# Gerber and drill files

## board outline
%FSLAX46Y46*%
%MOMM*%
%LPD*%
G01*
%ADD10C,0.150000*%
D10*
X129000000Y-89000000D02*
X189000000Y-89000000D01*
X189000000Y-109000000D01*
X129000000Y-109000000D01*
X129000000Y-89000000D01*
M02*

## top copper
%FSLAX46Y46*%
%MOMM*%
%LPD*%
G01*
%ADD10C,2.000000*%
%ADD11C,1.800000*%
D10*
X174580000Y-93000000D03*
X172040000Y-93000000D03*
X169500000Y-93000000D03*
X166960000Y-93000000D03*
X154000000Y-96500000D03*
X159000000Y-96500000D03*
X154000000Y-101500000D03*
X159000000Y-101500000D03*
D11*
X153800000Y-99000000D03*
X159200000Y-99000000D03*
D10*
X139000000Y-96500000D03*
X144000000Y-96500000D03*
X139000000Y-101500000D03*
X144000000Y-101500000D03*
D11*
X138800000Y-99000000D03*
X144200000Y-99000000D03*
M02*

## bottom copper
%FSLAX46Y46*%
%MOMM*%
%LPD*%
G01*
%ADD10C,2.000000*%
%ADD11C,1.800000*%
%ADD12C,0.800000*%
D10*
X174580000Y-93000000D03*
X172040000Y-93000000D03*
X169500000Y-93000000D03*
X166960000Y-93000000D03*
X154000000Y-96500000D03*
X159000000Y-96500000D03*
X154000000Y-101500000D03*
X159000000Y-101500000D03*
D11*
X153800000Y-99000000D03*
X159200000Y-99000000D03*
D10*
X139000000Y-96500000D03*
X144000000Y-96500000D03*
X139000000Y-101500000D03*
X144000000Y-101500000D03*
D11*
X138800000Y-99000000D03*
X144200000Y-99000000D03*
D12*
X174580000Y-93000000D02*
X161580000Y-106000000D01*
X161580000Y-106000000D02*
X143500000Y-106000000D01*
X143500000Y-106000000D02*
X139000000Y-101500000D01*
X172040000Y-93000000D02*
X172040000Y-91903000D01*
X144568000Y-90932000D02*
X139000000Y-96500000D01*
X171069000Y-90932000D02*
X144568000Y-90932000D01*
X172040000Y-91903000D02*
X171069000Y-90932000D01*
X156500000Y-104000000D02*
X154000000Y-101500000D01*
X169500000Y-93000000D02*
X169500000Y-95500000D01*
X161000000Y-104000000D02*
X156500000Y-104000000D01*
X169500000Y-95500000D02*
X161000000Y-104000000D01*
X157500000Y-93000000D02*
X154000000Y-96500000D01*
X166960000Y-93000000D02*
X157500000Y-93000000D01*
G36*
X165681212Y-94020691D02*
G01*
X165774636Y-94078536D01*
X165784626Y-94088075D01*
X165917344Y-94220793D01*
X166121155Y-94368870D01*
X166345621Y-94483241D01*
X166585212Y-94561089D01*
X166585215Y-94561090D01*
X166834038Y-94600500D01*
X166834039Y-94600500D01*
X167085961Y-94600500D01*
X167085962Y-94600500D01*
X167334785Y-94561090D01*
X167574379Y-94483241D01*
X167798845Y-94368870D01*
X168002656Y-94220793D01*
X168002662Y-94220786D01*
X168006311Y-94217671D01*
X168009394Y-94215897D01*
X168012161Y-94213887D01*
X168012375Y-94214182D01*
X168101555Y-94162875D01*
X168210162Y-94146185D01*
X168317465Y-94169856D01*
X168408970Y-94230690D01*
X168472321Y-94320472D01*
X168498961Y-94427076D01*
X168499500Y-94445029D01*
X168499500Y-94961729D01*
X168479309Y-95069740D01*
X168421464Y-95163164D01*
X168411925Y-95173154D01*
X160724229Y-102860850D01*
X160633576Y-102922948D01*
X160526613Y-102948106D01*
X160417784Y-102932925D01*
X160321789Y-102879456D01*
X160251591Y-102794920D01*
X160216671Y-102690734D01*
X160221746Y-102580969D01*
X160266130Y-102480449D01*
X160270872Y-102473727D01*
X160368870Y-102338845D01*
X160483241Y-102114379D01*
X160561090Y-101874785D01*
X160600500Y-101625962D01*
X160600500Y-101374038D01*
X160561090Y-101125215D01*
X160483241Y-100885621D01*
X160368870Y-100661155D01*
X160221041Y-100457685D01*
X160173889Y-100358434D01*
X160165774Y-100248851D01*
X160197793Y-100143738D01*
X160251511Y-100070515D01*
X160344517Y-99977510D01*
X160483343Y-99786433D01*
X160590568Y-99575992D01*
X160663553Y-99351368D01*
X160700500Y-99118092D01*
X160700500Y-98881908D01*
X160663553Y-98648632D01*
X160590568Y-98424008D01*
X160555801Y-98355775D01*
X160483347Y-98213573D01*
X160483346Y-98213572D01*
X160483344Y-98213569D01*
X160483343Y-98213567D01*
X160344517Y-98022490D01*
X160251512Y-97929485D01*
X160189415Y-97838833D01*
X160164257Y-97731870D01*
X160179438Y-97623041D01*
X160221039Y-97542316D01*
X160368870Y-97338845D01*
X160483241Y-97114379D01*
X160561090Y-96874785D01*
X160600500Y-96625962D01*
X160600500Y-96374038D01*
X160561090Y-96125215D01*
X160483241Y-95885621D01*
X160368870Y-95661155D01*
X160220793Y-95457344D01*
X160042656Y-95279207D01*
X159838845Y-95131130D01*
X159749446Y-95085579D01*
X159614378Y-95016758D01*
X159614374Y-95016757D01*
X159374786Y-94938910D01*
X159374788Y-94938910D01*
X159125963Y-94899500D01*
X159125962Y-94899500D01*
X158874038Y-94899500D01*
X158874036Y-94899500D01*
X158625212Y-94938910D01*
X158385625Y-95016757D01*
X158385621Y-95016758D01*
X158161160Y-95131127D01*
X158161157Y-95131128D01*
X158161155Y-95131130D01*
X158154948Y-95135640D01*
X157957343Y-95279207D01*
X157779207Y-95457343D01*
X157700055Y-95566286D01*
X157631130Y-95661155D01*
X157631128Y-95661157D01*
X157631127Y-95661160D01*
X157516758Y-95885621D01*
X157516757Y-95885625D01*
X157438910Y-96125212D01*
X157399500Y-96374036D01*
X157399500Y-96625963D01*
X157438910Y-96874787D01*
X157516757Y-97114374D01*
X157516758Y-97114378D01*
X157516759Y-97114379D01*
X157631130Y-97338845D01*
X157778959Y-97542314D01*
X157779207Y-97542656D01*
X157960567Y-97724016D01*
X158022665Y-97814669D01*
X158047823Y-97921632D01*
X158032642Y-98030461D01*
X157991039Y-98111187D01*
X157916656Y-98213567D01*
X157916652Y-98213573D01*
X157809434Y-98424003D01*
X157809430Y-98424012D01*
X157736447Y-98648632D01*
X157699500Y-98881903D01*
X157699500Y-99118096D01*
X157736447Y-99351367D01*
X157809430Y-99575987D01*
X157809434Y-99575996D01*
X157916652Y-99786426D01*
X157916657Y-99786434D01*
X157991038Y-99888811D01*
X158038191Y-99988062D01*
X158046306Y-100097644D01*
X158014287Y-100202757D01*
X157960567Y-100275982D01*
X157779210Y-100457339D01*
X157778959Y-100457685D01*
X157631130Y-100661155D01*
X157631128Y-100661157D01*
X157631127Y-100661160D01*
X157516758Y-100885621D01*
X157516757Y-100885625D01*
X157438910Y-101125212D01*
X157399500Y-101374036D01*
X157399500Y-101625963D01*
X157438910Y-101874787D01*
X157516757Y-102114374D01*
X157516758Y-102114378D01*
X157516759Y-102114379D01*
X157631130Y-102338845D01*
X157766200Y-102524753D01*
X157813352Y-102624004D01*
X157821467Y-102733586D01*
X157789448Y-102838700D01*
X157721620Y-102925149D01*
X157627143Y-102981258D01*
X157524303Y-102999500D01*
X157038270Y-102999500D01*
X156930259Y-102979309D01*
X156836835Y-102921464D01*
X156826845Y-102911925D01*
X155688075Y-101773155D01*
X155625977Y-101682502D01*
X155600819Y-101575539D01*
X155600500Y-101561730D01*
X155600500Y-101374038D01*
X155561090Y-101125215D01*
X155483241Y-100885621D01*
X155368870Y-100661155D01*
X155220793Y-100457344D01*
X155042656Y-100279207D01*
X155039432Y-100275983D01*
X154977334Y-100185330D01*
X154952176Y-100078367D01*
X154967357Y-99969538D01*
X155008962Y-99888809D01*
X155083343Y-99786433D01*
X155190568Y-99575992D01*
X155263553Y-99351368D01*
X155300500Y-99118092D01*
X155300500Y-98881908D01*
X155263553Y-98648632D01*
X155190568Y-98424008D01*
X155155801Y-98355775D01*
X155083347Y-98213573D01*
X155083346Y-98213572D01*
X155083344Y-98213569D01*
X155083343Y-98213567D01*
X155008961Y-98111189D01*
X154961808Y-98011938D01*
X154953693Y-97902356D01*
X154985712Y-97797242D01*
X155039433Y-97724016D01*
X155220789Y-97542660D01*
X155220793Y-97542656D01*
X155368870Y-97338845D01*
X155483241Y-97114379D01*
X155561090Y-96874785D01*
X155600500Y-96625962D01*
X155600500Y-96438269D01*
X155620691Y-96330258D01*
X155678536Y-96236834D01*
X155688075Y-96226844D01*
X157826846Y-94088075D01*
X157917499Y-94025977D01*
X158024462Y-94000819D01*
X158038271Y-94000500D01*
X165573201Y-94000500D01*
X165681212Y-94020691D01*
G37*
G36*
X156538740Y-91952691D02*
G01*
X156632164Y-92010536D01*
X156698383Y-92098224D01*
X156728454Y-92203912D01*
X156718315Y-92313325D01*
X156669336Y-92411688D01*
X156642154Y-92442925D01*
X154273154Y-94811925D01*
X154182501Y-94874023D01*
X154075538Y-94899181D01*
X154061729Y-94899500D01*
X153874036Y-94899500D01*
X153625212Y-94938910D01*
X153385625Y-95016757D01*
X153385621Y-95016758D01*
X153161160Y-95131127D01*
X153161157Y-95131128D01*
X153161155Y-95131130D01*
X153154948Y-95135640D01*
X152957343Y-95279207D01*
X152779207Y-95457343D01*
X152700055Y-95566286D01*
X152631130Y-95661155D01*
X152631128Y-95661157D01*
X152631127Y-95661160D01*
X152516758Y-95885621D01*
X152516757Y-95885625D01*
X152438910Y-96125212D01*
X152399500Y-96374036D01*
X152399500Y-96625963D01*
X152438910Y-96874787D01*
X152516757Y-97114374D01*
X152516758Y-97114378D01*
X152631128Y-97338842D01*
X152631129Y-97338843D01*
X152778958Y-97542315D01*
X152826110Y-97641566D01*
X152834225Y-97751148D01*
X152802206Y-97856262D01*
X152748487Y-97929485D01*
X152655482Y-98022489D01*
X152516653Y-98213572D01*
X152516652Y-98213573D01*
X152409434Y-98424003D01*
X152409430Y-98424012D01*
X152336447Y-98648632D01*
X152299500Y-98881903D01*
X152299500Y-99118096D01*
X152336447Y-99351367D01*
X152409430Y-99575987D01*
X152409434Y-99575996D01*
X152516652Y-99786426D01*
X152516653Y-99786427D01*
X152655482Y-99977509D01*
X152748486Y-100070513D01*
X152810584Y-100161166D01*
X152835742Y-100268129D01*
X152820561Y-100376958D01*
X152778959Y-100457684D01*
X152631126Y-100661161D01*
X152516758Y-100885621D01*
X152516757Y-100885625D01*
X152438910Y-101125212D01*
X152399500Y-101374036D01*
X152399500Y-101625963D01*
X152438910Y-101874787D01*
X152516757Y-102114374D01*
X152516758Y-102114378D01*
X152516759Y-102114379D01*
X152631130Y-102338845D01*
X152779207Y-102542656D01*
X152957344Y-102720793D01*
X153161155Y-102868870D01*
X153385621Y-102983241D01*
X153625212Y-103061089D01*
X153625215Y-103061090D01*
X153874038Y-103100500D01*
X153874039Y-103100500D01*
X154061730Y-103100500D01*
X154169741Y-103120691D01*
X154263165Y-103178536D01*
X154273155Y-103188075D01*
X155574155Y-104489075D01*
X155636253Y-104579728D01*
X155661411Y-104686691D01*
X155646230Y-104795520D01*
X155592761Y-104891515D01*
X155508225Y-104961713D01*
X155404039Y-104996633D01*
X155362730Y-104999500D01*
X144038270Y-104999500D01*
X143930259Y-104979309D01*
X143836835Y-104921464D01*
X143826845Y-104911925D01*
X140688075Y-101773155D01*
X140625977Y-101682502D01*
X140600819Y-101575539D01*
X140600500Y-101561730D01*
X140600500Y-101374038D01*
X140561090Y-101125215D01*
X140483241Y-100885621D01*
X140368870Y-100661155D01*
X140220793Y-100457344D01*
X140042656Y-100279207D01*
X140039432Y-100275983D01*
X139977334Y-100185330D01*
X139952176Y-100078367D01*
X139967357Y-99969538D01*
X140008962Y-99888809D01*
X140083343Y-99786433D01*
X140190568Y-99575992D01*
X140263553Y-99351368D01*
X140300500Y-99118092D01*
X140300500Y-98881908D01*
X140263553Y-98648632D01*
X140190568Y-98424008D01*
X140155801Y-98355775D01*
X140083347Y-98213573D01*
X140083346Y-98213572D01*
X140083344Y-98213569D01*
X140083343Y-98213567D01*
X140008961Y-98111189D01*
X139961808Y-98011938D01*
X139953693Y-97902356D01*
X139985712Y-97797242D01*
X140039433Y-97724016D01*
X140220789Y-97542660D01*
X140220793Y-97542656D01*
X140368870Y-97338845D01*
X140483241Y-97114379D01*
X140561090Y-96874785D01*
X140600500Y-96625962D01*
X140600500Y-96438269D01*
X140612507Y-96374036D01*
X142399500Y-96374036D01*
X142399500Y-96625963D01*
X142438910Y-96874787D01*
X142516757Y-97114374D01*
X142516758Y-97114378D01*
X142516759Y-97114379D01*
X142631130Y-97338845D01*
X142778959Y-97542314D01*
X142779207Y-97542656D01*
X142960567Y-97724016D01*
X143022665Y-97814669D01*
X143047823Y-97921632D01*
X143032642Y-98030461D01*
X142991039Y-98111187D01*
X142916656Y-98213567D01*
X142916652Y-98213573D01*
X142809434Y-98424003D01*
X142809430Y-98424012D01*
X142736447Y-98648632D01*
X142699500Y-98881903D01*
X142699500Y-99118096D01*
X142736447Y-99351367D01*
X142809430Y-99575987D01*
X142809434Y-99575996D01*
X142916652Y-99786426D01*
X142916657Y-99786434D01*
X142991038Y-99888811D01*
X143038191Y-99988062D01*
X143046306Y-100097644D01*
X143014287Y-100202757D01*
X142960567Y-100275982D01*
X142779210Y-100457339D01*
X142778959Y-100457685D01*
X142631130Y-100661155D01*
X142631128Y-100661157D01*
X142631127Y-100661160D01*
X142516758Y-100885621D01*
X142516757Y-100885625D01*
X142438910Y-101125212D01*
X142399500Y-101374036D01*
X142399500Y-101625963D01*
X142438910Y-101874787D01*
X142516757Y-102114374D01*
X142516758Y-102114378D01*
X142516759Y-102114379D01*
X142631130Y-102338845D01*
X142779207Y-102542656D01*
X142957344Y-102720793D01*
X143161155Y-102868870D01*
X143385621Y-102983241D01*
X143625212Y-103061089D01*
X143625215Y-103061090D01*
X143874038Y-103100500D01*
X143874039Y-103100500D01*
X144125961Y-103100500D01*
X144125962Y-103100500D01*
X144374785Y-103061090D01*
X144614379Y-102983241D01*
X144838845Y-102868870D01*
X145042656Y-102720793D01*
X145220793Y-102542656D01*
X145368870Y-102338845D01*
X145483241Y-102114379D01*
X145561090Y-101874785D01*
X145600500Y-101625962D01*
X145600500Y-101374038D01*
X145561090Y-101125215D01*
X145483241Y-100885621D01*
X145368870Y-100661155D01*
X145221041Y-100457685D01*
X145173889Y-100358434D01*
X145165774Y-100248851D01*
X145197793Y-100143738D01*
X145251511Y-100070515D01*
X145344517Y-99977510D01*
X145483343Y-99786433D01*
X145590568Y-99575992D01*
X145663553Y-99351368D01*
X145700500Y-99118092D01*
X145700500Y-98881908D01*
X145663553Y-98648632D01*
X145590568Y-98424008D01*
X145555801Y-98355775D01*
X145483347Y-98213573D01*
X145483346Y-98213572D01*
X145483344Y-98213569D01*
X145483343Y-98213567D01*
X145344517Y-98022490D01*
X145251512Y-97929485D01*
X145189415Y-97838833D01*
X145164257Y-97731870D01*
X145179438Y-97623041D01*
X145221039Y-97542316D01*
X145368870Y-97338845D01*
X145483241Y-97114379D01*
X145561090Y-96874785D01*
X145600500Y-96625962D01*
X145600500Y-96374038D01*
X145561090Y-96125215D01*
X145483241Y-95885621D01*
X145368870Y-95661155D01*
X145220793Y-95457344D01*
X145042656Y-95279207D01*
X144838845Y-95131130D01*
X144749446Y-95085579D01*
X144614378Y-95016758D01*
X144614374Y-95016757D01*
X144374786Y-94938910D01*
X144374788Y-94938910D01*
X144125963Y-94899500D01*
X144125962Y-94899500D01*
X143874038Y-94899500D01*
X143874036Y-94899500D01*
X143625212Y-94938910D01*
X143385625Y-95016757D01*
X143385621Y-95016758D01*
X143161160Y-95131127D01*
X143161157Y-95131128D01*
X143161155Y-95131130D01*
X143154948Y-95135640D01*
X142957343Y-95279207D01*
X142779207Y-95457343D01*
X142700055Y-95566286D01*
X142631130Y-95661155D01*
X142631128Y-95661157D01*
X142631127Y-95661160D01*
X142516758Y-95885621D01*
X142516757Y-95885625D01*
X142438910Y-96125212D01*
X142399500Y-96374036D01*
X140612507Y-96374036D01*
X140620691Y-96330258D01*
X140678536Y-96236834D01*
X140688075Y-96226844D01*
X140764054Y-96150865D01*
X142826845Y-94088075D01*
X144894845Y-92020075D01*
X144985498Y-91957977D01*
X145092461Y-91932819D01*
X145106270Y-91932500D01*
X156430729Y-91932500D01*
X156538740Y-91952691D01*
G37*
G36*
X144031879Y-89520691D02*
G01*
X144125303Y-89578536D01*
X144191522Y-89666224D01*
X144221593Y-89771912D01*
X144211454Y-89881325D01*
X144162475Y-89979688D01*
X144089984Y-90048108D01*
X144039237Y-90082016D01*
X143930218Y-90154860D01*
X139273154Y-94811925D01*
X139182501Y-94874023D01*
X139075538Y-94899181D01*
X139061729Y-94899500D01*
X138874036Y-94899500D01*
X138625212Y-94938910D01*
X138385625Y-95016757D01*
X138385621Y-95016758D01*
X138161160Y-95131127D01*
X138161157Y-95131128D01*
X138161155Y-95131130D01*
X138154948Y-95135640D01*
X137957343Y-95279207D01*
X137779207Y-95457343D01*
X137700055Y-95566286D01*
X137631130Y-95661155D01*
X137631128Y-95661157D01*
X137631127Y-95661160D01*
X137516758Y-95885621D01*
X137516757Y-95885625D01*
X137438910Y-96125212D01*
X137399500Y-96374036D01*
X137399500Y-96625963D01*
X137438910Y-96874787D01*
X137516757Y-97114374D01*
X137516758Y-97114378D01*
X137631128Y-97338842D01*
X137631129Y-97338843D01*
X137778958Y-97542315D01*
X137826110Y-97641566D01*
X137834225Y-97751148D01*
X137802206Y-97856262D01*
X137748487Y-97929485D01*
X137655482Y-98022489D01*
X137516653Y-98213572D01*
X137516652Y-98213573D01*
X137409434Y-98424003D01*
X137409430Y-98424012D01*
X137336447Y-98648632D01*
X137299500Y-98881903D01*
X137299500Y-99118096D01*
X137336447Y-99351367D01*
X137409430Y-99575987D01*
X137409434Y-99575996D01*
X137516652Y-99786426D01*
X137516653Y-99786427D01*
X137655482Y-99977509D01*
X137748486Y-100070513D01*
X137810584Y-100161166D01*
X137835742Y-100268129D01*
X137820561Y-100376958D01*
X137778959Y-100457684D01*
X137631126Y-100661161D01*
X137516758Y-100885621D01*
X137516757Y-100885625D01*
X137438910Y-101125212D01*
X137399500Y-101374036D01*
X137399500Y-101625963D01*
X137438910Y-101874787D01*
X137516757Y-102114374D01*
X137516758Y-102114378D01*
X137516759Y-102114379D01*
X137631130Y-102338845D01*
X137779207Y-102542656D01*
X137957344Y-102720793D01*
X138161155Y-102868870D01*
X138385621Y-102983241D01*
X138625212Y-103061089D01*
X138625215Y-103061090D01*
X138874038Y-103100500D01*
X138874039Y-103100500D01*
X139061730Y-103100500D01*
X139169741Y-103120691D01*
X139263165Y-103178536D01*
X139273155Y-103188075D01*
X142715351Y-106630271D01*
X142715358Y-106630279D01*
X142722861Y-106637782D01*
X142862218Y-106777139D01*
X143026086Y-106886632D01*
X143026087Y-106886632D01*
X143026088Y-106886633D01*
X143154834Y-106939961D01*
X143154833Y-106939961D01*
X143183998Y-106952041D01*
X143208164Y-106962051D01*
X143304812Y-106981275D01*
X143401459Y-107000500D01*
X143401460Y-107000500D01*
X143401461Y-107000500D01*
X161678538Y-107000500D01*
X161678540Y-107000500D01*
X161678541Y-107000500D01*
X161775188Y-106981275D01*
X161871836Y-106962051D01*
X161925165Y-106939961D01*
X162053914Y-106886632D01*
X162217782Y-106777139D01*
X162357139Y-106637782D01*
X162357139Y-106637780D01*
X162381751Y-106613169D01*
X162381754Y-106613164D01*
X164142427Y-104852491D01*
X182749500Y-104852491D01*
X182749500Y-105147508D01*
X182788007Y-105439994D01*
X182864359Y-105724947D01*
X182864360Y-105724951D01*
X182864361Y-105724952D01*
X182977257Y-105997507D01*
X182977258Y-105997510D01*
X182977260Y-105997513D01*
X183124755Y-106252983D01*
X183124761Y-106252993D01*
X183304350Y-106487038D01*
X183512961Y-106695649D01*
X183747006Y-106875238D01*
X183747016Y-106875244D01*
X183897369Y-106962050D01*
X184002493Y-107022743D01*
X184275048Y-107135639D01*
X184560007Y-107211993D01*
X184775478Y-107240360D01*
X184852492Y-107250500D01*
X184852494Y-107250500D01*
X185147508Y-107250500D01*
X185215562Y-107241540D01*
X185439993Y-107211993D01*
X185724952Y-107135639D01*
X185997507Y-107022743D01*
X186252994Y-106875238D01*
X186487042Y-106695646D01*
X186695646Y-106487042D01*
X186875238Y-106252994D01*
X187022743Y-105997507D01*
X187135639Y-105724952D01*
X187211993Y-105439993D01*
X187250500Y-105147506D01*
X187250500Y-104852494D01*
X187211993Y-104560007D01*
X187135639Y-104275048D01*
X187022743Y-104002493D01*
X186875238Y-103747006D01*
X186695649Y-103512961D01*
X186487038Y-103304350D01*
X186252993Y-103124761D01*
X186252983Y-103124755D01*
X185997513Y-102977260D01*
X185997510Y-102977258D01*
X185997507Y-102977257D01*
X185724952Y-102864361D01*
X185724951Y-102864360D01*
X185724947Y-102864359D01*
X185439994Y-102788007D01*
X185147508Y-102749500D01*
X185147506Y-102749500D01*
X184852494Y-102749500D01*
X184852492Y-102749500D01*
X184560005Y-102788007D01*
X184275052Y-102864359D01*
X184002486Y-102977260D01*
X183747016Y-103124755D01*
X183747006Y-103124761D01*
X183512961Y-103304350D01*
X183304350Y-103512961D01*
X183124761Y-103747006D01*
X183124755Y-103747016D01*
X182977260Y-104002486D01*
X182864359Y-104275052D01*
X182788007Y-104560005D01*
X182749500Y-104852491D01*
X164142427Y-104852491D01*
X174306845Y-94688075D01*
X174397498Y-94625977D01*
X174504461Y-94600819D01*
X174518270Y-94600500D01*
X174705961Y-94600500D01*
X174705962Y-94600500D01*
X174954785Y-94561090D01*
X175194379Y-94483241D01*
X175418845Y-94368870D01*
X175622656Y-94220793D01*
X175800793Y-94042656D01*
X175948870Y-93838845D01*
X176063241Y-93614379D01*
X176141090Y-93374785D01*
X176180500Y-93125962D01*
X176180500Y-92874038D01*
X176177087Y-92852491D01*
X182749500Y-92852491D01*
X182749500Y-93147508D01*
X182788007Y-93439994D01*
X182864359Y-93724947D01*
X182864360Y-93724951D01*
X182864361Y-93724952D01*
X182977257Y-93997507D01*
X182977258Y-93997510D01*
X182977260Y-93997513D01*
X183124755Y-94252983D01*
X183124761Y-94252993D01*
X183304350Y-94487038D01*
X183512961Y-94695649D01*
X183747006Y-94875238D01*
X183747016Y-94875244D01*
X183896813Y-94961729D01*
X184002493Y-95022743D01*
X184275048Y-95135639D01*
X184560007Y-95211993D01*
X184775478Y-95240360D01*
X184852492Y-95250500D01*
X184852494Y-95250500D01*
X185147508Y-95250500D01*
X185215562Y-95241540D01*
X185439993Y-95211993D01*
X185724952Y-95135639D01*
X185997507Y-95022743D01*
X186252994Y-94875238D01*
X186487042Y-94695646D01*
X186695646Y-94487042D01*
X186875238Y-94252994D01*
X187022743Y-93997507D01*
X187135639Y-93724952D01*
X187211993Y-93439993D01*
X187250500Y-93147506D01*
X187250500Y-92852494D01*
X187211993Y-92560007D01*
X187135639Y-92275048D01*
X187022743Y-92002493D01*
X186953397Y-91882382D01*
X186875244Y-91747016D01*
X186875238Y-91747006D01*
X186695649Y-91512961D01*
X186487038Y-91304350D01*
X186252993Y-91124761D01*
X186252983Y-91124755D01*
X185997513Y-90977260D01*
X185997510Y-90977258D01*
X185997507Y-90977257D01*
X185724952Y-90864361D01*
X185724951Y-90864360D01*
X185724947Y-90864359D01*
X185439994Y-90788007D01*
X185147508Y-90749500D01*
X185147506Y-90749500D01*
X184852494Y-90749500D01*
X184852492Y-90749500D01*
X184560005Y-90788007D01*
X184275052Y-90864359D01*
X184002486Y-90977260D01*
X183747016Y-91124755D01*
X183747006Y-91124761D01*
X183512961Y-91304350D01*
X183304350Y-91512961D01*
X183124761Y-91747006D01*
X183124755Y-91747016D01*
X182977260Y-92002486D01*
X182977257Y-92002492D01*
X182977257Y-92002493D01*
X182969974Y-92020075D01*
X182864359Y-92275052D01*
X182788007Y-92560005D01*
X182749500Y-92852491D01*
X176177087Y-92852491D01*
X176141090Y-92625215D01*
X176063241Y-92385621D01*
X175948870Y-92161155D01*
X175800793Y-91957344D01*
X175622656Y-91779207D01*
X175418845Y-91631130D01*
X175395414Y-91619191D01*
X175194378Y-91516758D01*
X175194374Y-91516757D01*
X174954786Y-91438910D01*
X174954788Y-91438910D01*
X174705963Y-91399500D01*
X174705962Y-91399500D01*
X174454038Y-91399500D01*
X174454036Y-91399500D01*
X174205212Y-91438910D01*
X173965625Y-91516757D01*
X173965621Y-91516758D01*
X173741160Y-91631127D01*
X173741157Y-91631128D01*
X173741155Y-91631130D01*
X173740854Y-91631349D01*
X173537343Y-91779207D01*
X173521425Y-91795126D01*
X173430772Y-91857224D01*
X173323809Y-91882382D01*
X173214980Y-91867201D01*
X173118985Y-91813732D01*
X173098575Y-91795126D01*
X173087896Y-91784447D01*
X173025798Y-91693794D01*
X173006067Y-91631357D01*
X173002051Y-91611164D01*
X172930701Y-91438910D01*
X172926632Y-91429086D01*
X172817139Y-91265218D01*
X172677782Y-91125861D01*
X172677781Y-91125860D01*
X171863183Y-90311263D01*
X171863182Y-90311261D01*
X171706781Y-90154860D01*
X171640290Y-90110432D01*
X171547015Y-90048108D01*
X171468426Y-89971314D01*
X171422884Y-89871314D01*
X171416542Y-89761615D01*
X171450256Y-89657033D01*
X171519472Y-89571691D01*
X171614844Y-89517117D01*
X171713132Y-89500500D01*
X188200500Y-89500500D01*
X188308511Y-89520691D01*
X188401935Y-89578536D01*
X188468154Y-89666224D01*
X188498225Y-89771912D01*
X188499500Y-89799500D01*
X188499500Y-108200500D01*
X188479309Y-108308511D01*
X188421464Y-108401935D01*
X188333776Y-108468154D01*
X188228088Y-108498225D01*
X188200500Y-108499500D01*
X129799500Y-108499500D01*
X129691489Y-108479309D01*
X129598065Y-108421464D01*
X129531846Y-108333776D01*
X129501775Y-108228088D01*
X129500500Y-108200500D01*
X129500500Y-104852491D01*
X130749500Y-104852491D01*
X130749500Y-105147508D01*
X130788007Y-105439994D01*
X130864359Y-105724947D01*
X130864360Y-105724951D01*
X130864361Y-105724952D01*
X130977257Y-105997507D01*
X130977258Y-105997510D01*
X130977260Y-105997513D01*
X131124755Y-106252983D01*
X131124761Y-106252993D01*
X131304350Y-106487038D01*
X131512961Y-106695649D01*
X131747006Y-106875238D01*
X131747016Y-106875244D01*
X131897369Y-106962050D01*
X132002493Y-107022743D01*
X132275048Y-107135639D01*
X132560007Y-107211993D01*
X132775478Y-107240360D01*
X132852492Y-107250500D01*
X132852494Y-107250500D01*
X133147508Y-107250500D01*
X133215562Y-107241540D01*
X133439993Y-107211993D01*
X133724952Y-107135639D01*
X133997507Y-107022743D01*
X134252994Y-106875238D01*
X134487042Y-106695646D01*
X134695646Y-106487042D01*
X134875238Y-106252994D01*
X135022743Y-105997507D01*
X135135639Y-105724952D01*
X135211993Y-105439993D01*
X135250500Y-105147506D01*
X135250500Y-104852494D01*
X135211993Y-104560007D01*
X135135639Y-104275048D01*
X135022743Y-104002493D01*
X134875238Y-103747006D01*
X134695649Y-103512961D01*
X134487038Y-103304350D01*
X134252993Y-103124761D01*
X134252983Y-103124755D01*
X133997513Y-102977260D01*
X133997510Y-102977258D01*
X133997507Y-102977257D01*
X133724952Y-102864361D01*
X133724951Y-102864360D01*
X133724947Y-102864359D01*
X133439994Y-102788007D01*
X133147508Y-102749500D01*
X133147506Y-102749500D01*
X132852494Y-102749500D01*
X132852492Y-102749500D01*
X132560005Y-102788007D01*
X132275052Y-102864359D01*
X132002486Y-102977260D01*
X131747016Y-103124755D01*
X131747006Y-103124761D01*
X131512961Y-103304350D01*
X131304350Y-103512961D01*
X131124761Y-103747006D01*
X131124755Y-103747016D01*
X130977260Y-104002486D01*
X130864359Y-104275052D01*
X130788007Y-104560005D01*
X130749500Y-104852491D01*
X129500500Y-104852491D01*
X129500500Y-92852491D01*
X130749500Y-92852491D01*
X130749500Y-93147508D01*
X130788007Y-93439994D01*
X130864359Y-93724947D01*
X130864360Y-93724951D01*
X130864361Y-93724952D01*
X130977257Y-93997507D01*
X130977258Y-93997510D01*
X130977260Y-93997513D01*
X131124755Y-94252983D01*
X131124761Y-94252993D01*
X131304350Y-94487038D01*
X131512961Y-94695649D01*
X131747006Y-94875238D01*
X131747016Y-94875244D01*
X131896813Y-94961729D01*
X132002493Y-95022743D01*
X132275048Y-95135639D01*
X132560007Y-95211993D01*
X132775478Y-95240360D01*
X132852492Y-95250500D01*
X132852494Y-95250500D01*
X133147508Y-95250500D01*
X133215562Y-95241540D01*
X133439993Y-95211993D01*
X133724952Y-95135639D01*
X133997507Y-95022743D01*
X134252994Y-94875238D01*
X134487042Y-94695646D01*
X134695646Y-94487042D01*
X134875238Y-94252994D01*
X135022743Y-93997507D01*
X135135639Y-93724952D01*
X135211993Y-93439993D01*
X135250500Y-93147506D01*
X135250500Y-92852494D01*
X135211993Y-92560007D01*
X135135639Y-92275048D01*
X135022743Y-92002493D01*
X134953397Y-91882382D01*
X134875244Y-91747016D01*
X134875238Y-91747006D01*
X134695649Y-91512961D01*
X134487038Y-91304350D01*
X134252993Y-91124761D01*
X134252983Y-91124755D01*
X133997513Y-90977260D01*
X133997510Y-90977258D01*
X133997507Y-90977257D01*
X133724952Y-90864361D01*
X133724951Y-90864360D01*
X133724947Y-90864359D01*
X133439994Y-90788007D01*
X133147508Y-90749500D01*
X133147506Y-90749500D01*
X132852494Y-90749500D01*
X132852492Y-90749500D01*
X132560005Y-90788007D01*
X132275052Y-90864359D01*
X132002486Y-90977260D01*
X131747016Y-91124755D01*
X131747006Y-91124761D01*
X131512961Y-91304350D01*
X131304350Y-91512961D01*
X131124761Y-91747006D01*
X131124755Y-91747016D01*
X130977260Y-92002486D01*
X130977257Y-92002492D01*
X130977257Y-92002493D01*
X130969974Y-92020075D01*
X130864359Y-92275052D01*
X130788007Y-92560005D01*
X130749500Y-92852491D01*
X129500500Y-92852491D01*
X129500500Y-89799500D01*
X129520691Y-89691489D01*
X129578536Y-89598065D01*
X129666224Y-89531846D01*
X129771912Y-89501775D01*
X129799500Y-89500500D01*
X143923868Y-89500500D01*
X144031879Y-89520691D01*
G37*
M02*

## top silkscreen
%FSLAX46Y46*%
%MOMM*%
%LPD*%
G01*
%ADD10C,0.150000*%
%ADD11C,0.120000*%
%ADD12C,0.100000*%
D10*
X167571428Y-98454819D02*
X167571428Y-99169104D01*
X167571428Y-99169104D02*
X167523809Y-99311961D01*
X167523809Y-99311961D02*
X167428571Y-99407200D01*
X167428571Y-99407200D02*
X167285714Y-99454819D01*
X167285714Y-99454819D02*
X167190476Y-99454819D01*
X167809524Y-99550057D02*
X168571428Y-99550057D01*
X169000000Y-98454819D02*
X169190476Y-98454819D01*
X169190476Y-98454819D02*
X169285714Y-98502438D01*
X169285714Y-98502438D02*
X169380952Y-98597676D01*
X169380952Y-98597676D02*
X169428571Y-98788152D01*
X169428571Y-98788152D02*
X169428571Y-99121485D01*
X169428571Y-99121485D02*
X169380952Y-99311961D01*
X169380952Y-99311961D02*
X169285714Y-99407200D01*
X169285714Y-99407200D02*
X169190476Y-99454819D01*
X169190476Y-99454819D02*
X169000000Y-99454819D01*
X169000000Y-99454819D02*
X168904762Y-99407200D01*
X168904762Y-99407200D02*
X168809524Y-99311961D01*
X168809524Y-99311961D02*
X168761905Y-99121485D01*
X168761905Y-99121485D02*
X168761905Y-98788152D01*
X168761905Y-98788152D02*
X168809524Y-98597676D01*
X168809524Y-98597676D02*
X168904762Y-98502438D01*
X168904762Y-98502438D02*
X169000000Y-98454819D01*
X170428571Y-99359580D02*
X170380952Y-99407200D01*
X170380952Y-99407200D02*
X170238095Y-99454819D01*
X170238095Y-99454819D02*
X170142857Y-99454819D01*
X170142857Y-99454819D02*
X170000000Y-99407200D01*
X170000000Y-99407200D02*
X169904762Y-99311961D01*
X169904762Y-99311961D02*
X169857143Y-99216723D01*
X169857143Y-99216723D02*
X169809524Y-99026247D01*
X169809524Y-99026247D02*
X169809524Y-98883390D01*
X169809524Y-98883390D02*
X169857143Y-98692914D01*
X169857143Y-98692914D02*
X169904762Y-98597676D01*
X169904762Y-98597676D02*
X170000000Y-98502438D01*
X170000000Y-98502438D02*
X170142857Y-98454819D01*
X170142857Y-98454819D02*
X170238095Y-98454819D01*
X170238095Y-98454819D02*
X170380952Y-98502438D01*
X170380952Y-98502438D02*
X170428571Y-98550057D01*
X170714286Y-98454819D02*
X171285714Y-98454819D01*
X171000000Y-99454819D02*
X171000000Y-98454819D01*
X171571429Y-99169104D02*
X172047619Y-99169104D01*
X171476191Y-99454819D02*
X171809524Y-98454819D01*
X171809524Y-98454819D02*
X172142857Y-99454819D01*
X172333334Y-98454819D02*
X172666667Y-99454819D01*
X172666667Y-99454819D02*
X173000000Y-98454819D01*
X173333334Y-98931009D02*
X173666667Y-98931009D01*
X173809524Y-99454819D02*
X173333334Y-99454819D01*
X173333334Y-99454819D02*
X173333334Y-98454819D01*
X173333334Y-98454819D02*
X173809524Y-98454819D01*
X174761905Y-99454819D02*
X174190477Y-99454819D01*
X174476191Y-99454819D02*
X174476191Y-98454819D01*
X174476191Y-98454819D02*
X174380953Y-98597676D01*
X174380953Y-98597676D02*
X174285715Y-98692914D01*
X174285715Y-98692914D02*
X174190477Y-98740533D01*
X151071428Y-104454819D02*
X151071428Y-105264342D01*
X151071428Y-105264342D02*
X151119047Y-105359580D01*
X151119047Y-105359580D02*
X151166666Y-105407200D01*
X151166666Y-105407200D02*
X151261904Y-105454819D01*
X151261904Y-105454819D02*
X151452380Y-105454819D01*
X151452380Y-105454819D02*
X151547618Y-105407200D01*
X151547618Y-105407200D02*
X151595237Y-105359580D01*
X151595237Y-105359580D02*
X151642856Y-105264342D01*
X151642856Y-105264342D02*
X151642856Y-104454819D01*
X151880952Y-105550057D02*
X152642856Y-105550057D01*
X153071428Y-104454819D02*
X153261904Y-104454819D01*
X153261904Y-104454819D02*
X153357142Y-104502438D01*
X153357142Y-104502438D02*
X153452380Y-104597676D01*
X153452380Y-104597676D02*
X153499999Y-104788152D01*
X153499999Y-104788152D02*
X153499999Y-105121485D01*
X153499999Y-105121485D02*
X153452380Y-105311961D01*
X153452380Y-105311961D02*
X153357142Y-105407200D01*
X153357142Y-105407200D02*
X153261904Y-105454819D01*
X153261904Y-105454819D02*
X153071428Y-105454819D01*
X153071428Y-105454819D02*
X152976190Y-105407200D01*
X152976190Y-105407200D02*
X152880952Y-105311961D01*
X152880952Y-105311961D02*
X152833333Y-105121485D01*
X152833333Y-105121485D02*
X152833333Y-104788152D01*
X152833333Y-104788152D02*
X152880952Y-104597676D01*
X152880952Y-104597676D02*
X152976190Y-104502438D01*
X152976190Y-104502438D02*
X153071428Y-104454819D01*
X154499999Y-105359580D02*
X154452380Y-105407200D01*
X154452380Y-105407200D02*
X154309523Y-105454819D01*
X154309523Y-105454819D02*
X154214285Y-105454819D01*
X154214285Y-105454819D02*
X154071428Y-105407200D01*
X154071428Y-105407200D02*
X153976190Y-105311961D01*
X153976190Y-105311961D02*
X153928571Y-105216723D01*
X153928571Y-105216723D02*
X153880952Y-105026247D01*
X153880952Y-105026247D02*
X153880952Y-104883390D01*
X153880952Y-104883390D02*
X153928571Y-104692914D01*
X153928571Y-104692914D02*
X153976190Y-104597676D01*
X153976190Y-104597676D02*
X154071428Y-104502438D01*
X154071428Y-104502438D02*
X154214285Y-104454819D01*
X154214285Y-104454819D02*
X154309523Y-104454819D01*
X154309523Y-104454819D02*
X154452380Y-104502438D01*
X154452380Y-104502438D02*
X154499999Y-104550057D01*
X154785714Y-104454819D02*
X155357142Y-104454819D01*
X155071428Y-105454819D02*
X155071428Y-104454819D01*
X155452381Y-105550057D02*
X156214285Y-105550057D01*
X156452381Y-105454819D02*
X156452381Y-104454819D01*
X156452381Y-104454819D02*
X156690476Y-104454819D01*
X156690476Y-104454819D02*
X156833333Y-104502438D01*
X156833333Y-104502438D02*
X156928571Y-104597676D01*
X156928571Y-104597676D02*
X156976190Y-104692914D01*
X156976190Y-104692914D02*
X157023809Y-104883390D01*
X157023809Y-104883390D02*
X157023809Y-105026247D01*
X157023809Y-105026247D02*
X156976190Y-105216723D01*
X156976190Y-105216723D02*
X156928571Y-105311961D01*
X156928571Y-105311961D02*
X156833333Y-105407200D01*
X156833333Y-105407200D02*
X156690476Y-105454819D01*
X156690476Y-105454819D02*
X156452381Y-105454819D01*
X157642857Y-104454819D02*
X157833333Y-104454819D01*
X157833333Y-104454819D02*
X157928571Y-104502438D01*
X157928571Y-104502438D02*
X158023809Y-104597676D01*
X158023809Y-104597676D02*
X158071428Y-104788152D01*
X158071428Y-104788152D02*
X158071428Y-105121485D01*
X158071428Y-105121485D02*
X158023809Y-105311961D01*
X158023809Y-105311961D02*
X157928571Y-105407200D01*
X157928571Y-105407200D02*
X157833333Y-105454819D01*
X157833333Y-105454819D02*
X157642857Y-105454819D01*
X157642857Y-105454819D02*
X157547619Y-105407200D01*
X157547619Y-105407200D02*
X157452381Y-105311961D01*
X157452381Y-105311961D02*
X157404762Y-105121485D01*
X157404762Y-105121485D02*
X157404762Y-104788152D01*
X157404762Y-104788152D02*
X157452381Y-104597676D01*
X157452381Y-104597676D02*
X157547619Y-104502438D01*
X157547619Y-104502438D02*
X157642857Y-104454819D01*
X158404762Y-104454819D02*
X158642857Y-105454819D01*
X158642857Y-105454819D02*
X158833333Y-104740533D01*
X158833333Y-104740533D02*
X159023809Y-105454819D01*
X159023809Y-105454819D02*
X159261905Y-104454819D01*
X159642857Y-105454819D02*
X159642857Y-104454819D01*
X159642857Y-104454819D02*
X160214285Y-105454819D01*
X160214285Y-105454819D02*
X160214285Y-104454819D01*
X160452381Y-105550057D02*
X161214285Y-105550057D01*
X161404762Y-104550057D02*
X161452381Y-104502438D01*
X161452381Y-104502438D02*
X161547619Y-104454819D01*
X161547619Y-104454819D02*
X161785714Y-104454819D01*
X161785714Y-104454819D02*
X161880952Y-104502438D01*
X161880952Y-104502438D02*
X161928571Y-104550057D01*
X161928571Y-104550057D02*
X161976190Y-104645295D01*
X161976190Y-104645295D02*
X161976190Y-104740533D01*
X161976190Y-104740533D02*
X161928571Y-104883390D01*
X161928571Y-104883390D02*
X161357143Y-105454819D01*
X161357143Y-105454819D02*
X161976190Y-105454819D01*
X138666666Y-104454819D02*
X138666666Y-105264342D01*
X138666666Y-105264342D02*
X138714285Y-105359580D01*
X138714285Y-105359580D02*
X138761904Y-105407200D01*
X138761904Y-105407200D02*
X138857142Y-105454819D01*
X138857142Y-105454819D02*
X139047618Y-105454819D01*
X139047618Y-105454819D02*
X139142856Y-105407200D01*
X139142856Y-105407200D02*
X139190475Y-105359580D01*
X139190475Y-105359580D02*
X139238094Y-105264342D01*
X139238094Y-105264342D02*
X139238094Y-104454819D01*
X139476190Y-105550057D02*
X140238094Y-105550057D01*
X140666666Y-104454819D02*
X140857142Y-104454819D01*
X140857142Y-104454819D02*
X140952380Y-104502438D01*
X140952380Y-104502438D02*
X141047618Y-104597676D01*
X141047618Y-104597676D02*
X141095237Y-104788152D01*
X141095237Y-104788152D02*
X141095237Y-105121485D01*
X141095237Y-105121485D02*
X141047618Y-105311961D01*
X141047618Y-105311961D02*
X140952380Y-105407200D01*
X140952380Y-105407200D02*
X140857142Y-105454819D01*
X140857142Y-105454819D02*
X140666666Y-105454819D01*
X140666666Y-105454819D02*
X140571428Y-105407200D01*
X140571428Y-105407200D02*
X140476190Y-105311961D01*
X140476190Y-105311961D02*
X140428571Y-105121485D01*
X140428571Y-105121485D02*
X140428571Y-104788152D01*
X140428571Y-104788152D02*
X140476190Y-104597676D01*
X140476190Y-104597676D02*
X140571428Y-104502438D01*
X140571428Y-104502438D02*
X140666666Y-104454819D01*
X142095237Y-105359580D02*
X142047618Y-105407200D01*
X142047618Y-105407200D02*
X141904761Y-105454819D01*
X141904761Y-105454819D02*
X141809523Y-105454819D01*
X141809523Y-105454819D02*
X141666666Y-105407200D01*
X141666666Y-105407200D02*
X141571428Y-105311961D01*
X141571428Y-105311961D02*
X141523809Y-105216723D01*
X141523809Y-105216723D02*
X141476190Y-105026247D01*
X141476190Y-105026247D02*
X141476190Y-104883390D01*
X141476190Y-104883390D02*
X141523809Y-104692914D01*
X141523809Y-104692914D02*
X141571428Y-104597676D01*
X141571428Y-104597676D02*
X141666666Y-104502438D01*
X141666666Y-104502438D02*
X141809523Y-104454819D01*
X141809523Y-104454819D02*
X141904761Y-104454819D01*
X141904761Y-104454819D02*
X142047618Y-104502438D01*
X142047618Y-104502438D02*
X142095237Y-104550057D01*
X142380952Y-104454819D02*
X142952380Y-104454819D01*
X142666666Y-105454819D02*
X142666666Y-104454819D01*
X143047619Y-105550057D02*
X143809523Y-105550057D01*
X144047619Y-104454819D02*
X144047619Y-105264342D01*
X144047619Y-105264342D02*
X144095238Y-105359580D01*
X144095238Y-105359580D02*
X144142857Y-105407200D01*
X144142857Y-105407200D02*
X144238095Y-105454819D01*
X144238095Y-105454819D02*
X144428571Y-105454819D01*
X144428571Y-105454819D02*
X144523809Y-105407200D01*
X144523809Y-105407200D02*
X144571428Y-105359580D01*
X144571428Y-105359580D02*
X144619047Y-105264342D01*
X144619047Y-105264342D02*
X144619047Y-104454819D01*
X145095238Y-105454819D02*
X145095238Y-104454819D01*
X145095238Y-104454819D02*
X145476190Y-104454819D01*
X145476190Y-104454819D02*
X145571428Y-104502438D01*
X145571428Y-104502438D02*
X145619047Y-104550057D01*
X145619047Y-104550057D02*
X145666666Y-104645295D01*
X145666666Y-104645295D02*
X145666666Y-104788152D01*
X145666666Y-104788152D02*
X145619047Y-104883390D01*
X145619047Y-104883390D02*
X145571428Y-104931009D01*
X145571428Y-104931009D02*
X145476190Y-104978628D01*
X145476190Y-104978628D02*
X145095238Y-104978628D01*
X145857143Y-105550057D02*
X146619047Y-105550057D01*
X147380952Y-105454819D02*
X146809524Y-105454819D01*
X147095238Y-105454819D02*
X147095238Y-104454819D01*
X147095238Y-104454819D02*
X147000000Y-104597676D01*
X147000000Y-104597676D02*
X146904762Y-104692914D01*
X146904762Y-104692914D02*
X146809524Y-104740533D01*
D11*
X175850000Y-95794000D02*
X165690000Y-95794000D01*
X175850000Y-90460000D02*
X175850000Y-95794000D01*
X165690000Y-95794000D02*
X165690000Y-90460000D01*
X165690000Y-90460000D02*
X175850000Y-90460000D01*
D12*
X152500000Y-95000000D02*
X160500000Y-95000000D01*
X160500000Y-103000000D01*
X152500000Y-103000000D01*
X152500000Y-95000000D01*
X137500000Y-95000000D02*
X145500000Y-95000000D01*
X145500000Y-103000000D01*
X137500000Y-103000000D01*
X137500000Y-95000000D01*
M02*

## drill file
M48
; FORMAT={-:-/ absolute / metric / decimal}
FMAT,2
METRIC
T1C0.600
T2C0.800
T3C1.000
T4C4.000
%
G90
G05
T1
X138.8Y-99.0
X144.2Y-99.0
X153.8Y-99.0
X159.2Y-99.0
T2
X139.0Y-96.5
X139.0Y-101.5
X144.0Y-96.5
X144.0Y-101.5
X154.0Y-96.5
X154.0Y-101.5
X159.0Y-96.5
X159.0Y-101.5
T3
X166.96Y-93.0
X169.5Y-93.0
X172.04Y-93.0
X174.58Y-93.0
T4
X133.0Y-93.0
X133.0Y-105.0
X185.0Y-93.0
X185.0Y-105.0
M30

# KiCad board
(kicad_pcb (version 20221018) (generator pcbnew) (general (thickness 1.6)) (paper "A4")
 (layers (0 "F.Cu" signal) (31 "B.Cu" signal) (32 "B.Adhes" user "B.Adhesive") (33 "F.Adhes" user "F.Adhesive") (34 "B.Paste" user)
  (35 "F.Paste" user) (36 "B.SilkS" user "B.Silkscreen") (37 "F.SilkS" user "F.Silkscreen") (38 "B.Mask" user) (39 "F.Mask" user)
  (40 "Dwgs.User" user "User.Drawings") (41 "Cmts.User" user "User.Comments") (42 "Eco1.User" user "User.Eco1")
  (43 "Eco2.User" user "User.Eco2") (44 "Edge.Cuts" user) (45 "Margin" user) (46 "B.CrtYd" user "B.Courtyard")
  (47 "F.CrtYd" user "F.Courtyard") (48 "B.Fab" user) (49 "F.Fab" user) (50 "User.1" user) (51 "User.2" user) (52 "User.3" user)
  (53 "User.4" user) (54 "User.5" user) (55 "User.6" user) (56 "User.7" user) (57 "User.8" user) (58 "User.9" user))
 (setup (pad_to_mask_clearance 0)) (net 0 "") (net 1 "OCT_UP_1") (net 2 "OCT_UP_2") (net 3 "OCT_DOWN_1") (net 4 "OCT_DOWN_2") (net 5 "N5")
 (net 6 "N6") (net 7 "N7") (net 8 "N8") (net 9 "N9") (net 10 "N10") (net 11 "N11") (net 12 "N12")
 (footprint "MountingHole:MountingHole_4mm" (layer "F.Cu") (at 185 93)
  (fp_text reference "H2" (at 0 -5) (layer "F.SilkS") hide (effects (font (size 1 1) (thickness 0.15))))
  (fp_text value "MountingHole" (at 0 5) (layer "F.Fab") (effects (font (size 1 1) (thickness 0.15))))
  (pad "" np_thru_hole circle (at 0 0) (size 4 4) (drill 4) (layers "*.Cu" "*.Mask")))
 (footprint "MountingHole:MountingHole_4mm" (layer "F.Cu") (at 133 105)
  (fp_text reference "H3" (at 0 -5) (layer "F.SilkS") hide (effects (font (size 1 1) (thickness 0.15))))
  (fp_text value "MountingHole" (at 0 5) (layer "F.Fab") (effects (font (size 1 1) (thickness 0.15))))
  (pad "" np_thru_hole circle (at 0 0) (size 4 4) (drill 4) (layers "*.Cu" "*.Mask")))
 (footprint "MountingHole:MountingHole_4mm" (layer "F.Cu") (at 133 93)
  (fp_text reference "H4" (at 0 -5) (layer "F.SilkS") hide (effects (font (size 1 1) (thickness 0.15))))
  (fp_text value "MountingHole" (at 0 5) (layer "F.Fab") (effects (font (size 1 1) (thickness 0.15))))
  (pad "" np_thru_hole circle (at 0 0) (size 4 4) (drill 4) (layers "*.Cu" "*.Mask")))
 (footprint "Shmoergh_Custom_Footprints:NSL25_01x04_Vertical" (layer "F.Cu") (at 174.58 93 180)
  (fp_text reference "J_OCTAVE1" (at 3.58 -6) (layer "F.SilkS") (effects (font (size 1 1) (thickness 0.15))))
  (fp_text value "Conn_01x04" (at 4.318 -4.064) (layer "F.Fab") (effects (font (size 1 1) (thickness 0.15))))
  (fp_line (start -1.27 -2.794) (end 8.89 -2.794) (stroke (width 0.12) (type solid)) (layer "F.SilkS"))
  (fp_line (start -1.27 2.54) (end -1.27 -2.794) (stroke (width 0.12) (type solid)) (layer "F.SilkS"))
  (fp_line (start 8.89 -2.794) (end 8.89 2.54) (stroke (width 0.12) (type solid)) (layer "F.SilkS"))
  (fp_line (start 8.89 2.54) (end -1.27 2.54) (stroke (width 0.12) (type solid)) (layer "F.SilkS"))
  (pad "1" thru_hole circle (at 0 0 180) (size 2 2) (drill 1) (layers "*.Cu" "*.Mask") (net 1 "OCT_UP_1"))
  (pad "2" thru_hole circle (at 2.54 0 180) (size 2 2) (drill 1) (layers "*.Cu" "*.Mask") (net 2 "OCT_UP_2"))
  (pad "3" thru_hole circle (at 5.08 0 180) (size 2 2) (drill 1) (layers "*.Cu" "*.Mask") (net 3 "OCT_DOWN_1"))
  (pad "4" thru_hole circle (at 7.62 0 180) (size 2 2) (drill 1) (layers "*.Cu" "*.Mask") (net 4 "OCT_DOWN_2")))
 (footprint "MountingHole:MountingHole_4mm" (layer "F.Cu") (at 185 105)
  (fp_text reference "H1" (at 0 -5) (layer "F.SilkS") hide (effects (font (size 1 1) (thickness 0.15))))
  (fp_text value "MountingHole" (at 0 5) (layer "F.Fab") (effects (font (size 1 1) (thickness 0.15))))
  (pad "" np_thru_hole circle (at 0 0) (size 4 4) (drill 4) (layers "*.Cu" "*.Mask")))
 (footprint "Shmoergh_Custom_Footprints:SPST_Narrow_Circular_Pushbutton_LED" (layer "F.Cu") (at 156.5 99)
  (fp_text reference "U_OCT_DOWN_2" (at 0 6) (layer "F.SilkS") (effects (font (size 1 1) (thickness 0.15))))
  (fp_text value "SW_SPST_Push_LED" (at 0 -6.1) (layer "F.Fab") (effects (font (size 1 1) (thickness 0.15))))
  (fp_rect (start -4 -4) (end 4 4) (stroke (width 0.1) (type default)) (fill none) (layer "F.SilkS"))
  (pad "1" thru_hole circle (at -2.5 -2.5) (size 2 2) (drill 0.8) (layers "*.Cu" "*.Mask") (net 4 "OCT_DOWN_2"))
  (pad "2" thru_hole circle (at 2.5 -2.5) (size 2 2) (drill 0.8) (layers "*.Cu" "*.Mask") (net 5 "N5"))
  (pad "3" thru_hole circle (at -2.5 2.5) (size 2 2) (drill 0.8) (layers "*.Cu" "*.Mask") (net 3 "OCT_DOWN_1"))
  (pad "4" thru_hole circle (at 2.5 2.5) (size 2 2) (drill 0.8) (layers "*.Cu" "*.Mask") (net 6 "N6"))
  (pad "L1" thru_hole circle (at -2.7 0) (size 1.8 1.8) (drill 0.6) (layers "*.Cu" "*.Mask") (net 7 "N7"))
  (pad "L2" thru_hole circle (at 2.7 0) (size 1.8 1.8) (drill 0.6) (layers "*.Cu" "*.Mask") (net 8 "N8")))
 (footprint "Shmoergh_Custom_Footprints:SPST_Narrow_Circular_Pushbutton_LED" (layer "F.Cu") (at 141.5 99)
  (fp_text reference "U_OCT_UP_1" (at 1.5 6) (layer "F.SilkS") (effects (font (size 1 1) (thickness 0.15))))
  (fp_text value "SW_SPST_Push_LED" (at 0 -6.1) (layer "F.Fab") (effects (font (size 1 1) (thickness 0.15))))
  (fp_rect (start -4 -4) (end 4 4) (stroke (width 0.1) (type default)) (fill none) (layer "F.SilkS"))
  (pad "1" thru_hole circle (at -2.5 -2.5) (size 2 2) (drill 0.8) (layers "*.Cu" "*.Mask") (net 2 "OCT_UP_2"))
  (pad "2" thru_hole circle (at 2.5 -2.5) (size 2 2) (drill 0.8) (layers "*.Cu" "*.Mask") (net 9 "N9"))
  (pad "3" thru_hole circle (at -2.5 2.5) (size 2 2) (drill 0.8) (layers "*.Cu" "*.Mask") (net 1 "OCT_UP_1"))
  (pad "4" thru_hole circle (at 2.5 2.5) (size 2 2) (drill 0.8) (layers "*.Cu" "*.Mask") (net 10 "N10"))
  (pad "L1" thru_hole circle (at -2.7 0) (size 1.8 1.8) (drill 0.6) (layers "*.Cu" "*.Mask") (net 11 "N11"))
  (pad "L2" thru_hole circle (at 2.7 0) (size 1.8 1.8) (drill 0.6) (layers "*.Cu" "*.Mask") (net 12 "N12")))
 (gr_rect (start 129 89) (end 189 109) (stroke (width 0.15) (type default)) (fill none) (layer "Edge.Cuts"))
 (segment (start 174.58 93) (end 161.58 106) (width 0.8) (layer "B.Cu") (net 1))
 (segment (start 161.58 106) (end 143.5 106) (width 0.8) (layer "B.Cu") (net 1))
 (segment (start 143.5 106) (end 139 101.5) (width 0.8) (layer "B.Cu") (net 1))
 (segment (start 172.04 93) (end 172.04 91.903) (width 0.8) (layer "B.Cu") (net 2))
 (segment (start 144.568 90.932) (end 139 96.5) (width 0.8) (layer "B.Cu") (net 2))
 (segment (start 171.069 90.932) (end 144.568 90.932) (width 0.8) (layer "B.Cu") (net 2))
 (segment (start 172.04 91.903) (end 171.069 90.932) (width 0.8) (layer "B.Cu") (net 2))
 (segment (start 156.5 104) (end 154 101.5) (width 0.8) (layer "B.Cu") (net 3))
 (segment (start 169.5 93) (end 169.5 95.5) (width 0.8) (layer "B.Cu") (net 3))
 (segment (start 161 104) (end 156.5 104) (width 0.8) (layer "B.Cu") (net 3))
 (segment (start 169.5 95.5) (end 161 104) (width 0.8) (layer "B.Cu") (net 3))
 (segment (start 157.5 93) (end 154 96.5) (width 0.8) (layer "B.Cu") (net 4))
 (segment (start 166.96 93) (end 157.5 93) (width 0.8) (layer "B.Cu") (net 4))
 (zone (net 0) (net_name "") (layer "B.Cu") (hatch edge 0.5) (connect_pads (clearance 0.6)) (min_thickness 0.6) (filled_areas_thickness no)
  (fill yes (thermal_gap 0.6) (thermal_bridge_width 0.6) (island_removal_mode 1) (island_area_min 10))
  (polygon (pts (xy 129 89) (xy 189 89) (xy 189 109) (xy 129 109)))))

